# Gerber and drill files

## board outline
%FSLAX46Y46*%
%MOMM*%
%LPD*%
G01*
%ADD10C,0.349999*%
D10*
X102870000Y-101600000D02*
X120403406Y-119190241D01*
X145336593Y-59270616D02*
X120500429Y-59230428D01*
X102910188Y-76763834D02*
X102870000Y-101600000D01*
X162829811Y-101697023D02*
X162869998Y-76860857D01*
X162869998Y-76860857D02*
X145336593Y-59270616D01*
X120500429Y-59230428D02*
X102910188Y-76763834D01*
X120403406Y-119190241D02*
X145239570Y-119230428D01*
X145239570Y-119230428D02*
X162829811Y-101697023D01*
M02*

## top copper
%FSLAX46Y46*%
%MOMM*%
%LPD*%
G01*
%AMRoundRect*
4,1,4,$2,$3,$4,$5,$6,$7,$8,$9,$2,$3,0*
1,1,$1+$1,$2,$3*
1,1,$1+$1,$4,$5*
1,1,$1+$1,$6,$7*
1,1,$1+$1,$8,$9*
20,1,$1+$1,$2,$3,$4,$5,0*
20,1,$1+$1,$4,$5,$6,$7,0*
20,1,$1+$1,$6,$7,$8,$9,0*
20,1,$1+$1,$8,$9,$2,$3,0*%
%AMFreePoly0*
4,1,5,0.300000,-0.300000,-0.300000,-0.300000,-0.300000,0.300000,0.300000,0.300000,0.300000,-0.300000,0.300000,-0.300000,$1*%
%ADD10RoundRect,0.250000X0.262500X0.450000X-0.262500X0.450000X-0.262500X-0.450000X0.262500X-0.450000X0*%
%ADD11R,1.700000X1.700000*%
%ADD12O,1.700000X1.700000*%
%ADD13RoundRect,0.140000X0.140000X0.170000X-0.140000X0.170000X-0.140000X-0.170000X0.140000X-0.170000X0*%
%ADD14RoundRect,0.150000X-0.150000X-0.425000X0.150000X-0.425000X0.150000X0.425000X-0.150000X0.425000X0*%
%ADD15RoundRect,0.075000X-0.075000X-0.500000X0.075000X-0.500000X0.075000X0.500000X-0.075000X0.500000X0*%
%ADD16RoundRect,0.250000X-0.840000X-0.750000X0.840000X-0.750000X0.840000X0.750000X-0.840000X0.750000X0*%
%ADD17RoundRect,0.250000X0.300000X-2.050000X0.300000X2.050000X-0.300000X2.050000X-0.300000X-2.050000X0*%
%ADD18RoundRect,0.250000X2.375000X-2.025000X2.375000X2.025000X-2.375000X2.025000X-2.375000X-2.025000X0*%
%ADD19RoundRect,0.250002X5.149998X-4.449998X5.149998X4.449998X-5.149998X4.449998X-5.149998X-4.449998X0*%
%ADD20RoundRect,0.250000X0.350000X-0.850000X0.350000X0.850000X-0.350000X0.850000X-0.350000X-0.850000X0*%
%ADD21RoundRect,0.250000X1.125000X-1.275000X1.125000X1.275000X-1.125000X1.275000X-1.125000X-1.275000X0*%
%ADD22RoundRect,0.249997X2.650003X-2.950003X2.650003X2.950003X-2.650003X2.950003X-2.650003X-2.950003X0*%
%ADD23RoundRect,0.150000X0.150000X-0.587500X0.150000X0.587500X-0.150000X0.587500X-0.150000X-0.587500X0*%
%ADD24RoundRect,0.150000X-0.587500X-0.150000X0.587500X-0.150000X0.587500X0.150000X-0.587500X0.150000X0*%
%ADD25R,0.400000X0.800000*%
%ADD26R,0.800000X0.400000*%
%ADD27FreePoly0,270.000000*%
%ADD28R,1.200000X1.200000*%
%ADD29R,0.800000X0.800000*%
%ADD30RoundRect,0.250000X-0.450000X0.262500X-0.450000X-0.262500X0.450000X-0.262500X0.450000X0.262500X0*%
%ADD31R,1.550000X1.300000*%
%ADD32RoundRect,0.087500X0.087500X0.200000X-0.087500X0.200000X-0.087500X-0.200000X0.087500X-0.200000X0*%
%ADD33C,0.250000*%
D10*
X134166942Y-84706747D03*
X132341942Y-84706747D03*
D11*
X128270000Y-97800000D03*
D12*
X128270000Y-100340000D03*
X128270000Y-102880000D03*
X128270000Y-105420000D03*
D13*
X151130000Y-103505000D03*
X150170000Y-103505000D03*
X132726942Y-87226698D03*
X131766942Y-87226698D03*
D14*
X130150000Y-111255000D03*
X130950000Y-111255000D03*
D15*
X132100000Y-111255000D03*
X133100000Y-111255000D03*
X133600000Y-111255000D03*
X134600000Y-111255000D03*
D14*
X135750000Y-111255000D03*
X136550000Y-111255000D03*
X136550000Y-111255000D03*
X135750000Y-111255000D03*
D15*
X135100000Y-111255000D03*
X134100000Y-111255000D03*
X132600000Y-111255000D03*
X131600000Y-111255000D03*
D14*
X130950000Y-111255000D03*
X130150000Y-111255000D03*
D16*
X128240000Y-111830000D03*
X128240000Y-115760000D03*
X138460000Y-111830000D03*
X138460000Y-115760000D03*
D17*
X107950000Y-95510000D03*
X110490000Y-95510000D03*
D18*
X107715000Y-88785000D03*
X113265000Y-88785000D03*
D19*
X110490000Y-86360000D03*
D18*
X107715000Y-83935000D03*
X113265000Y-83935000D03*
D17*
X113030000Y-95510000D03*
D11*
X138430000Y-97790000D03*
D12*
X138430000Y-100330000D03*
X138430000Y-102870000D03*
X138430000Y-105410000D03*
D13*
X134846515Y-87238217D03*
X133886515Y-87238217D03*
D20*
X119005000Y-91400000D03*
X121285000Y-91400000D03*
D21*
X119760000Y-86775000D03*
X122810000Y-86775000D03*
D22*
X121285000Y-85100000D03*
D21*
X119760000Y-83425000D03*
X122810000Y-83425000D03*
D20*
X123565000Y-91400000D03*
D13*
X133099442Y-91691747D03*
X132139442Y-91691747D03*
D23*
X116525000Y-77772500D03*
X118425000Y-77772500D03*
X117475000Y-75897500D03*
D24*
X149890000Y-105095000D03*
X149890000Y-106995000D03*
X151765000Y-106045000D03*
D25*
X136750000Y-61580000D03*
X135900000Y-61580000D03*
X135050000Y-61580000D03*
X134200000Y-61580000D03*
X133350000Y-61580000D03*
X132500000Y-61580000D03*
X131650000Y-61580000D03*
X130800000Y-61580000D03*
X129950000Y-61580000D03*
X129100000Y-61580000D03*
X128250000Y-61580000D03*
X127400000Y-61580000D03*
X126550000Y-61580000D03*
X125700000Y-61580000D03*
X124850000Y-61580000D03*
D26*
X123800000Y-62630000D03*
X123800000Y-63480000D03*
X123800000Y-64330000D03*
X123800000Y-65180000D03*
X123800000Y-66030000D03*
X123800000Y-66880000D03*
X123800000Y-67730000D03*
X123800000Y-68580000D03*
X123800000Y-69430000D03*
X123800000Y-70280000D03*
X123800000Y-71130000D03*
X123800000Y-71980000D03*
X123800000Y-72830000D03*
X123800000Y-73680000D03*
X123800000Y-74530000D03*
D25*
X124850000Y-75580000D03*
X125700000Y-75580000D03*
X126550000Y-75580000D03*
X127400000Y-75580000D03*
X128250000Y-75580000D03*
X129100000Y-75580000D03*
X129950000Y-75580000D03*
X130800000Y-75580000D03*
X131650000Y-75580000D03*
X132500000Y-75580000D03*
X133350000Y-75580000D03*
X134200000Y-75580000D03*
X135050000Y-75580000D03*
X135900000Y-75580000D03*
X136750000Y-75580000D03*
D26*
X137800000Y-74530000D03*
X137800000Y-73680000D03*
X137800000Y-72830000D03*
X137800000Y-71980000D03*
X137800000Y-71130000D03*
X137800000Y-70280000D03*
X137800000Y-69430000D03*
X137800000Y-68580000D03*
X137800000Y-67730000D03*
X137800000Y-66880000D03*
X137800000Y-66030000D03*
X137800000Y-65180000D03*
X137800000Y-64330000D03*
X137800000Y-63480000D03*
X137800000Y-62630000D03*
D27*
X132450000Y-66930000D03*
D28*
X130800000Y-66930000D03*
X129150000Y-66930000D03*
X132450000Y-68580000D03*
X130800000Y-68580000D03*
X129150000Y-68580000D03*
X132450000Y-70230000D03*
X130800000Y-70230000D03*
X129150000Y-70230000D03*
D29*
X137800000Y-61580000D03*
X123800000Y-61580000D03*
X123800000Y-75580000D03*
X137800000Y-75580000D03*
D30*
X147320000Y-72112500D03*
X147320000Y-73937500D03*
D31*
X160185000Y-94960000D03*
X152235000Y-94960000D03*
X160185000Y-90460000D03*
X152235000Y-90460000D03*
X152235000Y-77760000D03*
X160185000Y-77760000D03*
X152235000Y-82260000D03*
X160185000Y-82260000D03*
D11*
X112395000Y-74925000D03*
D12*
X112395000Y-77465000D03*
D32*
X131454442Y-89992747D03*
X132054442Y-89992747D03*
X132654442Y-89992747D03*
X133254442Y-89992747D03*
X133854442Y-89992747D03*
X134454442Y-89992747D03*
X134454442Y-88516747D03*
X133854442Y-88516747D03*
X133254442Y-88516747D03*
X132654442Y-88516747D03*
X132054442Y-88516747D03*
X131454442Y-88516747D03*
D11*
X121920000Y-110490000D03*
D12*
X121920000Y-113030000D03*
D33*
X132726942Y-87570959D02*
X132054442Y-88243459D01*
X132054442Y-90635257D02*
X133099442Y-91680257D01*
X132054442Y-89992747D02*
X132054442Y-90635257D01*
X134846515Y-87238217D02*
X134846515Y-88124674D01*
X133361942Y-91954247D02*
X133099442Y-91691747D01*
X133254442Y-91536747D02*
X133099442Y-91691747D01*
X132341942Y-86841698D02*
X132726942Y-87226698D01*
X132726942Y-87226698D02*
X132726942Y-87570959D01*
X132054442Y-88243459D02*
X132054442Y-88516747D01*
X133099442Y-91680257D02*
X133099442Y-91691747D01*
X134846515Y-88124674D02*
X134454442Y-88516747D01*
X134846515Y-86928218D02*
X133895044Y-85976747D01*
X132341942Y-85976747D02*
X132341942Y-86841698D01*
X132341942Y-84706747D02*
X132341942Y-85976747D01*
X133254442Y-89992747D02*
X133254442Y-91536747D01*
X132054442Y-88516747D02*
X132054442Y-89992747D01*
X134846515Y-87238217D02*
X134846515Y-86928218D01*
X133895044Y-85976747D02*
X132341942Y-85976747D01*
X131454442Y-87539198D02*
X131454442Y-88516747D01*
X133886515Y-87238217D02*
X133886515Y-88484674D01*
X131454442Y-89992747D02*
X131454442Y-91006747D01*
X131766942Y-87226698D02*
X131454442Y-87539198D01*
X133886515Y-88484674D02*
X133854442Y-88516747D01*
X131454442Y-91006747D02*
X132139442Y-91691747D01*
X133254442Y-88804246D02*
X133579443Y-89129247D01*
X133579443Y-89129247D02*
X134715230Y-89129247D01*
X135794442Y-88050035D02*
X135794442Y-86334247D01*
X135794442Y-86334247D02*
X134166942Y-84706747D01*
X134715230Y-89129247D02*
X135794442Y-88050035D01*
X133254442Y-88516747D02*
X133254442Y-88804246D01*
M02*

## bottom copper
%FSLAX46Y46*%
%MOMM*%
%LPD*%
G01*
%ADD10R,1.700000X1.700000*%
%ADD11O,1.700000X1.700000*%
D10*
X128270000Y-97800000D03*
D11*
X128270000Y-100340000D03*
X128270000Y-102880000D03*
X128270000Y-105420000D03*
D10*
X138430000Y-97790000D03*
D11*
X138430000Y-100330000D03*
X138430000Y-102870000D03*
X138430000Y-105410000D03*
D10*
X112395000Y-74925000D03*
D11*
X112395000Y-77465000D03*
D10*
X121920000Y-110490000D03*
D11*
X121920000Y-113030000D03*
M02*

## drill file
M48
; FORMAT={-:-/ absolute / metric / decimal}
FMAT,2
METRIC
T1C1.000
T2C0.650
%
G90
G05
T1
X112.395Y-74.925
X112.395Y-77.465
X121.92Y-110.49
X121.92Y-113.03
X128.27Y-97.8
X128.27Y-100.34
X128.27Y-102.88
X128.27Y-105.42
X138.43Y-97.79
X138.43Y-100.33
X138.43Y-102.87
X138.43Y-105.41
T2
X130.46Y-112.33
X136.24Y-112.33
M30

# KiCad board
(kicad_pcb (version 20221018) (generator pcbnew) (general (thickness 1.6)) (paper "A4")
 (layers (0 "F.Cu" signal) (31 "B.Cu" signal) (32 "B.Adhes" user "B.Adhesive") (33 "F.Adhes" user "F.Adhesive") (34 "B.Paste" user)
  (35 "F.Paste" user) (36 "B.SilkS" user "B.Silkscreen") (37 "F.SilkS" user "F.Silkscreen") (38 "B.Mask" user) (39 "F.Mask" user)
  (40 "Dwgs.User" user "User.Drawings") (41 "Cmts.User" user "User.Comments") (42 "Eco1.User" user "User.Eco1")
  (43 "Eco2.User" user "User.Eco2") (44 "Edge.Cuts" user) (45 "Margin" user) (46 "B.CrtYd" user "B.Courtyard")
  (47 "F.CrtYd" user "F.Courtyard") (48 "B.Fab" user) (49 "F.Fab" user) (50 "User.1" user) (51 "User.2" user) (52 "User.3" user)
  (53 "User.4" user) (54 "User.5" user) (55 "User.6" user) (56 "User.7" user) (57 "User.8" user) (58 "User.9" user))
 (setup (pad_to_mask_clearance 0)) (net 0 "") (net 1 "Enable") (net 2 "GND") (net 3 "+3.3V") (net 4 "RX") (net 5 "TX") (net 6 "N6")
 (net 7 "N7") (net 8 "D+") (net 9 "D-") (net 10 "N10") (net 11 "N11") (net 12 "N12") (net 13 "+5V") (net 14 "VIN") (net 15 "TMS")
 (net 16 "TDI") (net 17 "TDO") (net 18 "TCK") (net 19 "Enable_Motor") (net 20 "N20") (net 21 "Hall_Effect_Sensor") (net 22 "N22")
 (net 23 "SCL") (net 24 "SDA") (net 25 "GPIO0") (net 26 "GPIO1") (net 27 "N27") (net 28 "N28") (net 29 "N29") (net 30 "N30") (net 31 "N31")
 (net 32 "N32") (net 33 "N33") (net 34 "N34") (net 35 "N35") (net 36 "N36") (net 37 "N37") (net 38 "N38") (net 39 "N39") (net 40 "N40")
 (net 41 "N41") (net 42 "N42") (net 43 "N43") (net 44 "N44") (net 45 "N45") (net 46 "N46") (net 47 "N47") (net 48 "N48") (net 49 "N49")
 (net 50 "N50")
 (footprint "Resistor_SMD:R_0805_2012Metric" (layer "F.Cu") (at 133.254442 84.706747 180)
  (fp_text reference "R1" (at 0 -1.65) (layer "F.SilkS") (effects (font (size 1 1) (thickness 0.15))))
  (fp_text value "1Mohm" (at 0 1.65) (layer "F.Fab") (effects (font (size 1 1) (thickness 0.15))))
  (pad "1" smd roundrect (at -0.9125 0 180) (size 1.025 1.4) (layers "F.Cu" "F.Paste" "F.Mask") (roundrect_rratio 0.243902) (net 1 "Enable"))
  (pad "2" smd roundrect (at 0.9125 0 180) (size 1.025 1.4) (layers "F.Cu" "F.Paste" "F.Mask") (roundrect_rratio 0.243902) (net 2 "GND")))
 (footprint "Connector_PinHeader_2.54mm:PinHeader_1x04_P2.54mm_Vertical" (layer "F.Cu") (at 128.27 97.8)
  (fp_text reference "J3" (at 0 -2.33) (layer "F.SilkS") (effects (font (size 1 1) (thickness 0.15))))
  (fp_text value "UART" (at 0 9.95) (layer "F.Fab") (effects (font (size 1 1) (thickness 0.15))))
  (pad "1" thru_hole rect (at 0 0) (size 1.7 1.7) (drill 1) (layers "*.Cu" "*.Mask") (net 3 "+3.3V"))
  (pad "2" thru_hole oval (at 0 2.54) (size 1.7 1.7) (drill 1) (layers "*.Cu" "*.Mask") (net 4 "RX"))
  (pad "3" thru_hole oval (at 0 5.08) (size 1.7 1.7) (drill 1) (layers "*.Cu" "*.Mask") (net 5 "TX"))
  (pad "4" thru_hole oval (at 0 7.62) (size 1.7 1.7) (drill 1) (layers "*.Cu" "*.Mask") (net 2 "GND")))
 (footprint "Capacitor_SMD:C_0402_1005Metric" (layer "F.Cu") (at 150.65 103.505 180)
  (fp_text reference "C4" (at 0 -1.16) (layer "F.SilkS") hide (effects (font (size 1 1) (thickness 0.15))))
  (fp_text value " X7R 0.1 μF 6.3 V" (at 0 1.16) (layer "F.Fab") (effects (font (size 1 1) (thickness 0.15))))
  (pad "1" smd roundrect (at -0.48 0 180) (size 0.56 0.62) (layers "F.Cu" "F.Paste" "F.Mask") (roundrect_rratio 0.25) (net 2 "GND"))
  (pad "2" smd roundrect (at 0.48 0 180) (size 0.56 0.62) (layers "F.Cu" "F.Paste" "F.Mask") (roundrect_rratio 0.25) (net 3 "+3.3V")))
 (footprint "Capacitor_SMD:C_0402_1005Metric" (layer "F.Cu") (at 132.246942 87.226698 180)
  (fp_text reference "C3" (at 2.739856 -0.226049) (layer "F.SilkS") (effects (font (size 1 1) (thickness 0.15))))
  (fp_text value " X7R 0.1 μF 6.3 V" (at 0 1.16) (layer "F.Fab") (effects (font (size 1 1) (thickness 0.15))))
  (pad "1" smd roundrect (at -0.48 0 180) (size 0.56 0.62) (layers "F.Cu" "F.Paste" "F.Mask") (roundrect_rratio 0.25) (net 2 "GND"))
  (pad "2" smd roundrect (at 0.48 0 180) (size 0.56 0.62) (layers "F.Cu" "F.Paste" "F.Mask") (roundrect_rratio 0.25) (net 3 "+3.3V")))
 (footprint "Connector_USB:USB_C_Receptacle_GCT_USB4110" (layer "F.Cu") (at 133.35 114.935)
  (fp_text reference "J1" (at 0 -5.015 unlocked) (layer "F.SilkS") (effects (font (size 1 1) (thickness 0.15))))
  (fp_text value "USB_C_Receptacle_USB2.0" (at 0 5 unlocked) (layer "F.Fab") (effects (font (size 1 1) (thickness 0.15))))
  (pad "" np_thru_hole circle (at -2.89 -2.605) (size 0.65 0.65) (drill 0.65) (layers "F&B.Cu" "*.Mask"))
  (pad "" np_thru_hole circle (at 2.89 -2.605) (size 0.65 0.65) (drill 0.65) (layers "F&B.Cu" "*.Mask"))
  (pad "A1" smd roundrect (at -3.2 -3.68) (size 0.6 1.15) (layers "F.Cu" "F.Paste" "F.Mask") (roundrect_rratio 0.25) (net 2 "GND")
   (thermal_bridge_angle 45))
  (pad "A4" smd roundrect (at -2.4 -3.68) (size 0.6 1.15) (layers "F.Cu" "F.Paste" "F.Mask") (roundrect_rratio 0.25) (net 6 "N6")
   (thermal_bridge_angle 45))
  (pad "A5" smd roundrect (at -1.25 -3.68) (size 0.3 1.15) (layers "F.Cu" "F.Paste" "F.Mask") (roundrect_rratio 0.25) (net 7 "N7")
   (thermal_bridge_angle 45))
  (pad "A6" smd roundrect (at -0.25 -3.68) (size 0.3 1.15) (layers "F.Cu" "F.Paste" "F.Mask") (roundrect_rratio 0.25) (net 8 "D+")
   (thermal_bridge_angle 45))
  (pad "A7" smd roundrect (at 0.25 -3.68) (size 0.3 1.15) (layers "F.Cu" "F.Paste" "F.Mask") (roundrect_rratio 0.25) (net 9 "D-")
   (thermal_bridge_angle 45))
  (pad "A8" smd roundrect (at 1.25 -3.68) (size 0.3 1.15) (layers "F.Cu" "F.Paste" "F.Mask") (roundrect_rratio 0.25) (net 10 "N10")
   (thermal_bridge_angle 45))
  (pad "A9" smd roundrect (at 2.4 -3.68) (size 0.6 1.15) (layers "F.Cu" "F.Paste" "F.Mask") (roundrect_rratio 0.25) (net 6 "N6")
   (thermal_bridge_angle 45))
  (pad "A12" smd roundrect (at 3.2 -3.68) (size 0.6 1.15) (layers "F.Cu" "F.Paste" "F.Mask") (roundrect_rratio 0.25) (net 2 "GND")
   (thermal_bridge_angle 45))
  (pad "B1" smd roundrect (at 3.2 -3.68) (size 0.6 1.15) (layers "F.Cu" "F.Paste" "F.Mask") (roundrect_rratio 0.25) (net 2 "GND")
   (thermal_bridge_angle 45))
  (pad "B4" smd roundrect (at 2.4 -3.68) (size 0.6 1.15) (layers "F.Cu" "F.Paste" "F.Mask") (roundrect_rratio 0.25) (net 6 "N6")
   (thermal_bridge_angle 45))
  (pad "B5" smd roundrect (at 1.75 -3.68) (size 0.3 1.15) (layers "F.Cu" "F.Paste" "F.Mask") (roundrect_rratio 0.25) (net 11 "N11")
   (thermal_bridge_angle 45))
  (pad "B6" smd roundrect (at 0.75 -3.68) (size 0.3 1.15) (layers "F.Cu" "F.Paste" "F.Mask") (roundrect_rratio 0.25) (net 8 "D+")
   (thermal_bridge_angle 45))
  (pad "B7" smd roundrect (at -0.75 -3.68) (size 0.3 1.15) (layers "F.Cu" "F.Paste" "F.Mask") (roundrect_rratio 0.25) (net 9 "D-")
   (thermal_bridge_angle 45))
  (pad "B8" smd roundrect (at -1.75 -3.68) (size 0.3 1.15) (layers "F.Cu" "F.Paste" "F.Mask") (roundrect_rratio 0.25) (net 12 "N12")
   (thermal_bridge_angle 45))
  (pad "B9" smd roundrect (at -2.4 -3.68) (size 0.6 1.15) (layers "F.Cu" "F.Paste" "F.Mask") (roundrect_rratio 0.25) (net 6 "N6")
   (thermal_bridge_angle 45))
  (pad "B12" smd roundrect (at -3.2 -3.68) (size 0.6 1.15) (layers "F.Cu" "F.Paste" "F.Mask") (roundrect_rratio 0.25) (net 2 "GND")
   (thermal_bridge_angle 45))
  (pad "S1" smd roundrect (at -5.11 -3.105) (size 2.18 2) (layers "F.Cu" "F.Paste" "F.Mask") (roundrect_rratio 0.125) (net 2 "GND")
   (thermal_bridge_angle 45))
  (pad "S1" smd roundrect (at -5.11 0.825) (size 2.18 2) (layers "F.Cu" "F.Paste" "F.Mask") (roundrect_rratio 0.125) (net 2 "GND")
   (thermal_bridge_angle 45))
  (pad "S1" smd roundrect (at 5.11 -3.105) (size 2.18 2) (layers "F.Cu" "F.Paste" "F.Mask") (roundrect_rratio 0.125) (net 2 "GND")
   (thermal_bridge_angle 45))
  (pad "S1" smd roundrect (at 5.11 0.825) (size 2.18 2) (layers "F.Cu" "F.Paste" "F.Mask") (roundrect_rratio 0.125) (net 2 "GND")
   (thermal_bridge_angle 45)))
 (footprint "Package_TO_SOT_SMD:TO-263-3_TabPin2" (layer "F.Cu") (at 110.49 87.86 90)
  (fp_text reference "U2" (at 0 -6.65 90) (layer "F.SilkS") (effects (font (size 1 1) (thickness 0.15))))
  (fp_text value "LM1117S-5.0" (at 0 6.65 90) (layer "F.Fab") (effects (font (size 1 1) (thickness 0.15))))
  (pad "1" smd roundrect (at -7.65 -2.54 90) (size 4.6 1.1) (layers "F.Cu" "F.Paste" "F.Mask") (roundrect_rratio 0.227273) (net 2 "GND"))
  (pad "2" smd roundrect (at -7.65 0 90) (size 4.6 1.1) (layers "F.Cu" "F.Paste" "F.Mask") (roundrect_rratio 0.227273) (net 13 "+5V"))
  (pad "2" smd roundrect (at -0.925 -2.775 90) (size 4.55 5.25) (layers "F.Cu" "F.Paste") (roundrect_rratio 0.054945) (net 13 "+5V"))
  (pad "2" smd roundrect (at -0.925 2.775 90) (size 4.55 5.25) (layers "F.Cu" "F.Paste") (roundrect_rratio 0.054945) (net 13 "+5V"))
  (pad "2" smd roundrect (at 1.5 0 90) (size 9.4 10.8) (layers "F.Cu" "F.Mask") (roundrect_rratio 0.026596) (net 13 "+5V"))
  (pad "2" smd roundrect (at 3.925 -2.775 90) (size 4.55 5.25) (layers "F.Cu" "F.Paste") (roundrect_rratio 0.054945) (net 13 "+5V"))
  (pad "2" smd roundrect (at 3.925 2.775 90) (size 4.55 5.25) (layers "F.Cu" "F.Paste") (roundrect_rratio 0.054945) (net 13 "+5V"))
  (pad "3" smd roundrect (at -7.65 2.54 90) (size 4.6 1.1) (layers "F.Cu" "F.Paste" "F.Mask") (roundrect_rratio 0.227273) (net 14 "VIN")))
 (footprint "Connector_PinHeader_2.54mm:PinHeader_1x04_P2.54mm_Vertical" (layer "F.Cu") (at 138.43 97.79)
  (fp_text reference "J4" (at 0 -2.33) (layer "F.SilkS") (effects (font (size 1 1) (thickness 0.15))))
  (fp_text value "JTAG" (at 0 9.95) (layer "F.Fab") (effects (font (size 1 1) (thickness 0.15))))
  (pad "1" thru_hole rect (at 0 0) (size 1.7 1.7) (drill 1) (layers "*.Cu" "*.Mask") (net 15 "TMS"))
  (pad "2" thru_hole oval (at 0 2.54) (size 1.7 1.7) (drill 1) (layers "*.Cu" "*.Mask") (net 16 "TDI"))
  (pad "3" thru_hole oval (at 0 5.08) (size 1.7 1.7) (drill 1) (layers "*.Cu" "*.Mask") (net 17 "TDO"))
  (pad "4" thru_hole oval (at 0 7.62) (size 1.7 1.7) (drill 1) (layers "*.Cu" "*.Mask") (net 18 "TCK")))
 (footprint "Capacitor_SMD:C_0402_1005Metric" (layer "F.Cu") (at 134.366515 87.238217 180)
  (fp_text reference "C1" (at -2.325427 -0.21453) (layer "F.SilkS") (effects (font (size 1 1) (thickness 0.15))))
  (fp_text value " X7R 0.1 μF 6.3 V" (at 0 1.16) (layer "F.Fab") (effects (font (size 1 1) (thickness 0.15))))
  (pad "1" smd roundrect (at -0.48 0 180) (size 0.56 0.62) (layers "F.Cu" "F.Paste" "F.Mask") (roundrect_rratio 0.25) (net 2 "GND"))
  (pad "2" smd roundrect (at 0.48 0 180) (size 0.56 0.62) (layers "F.Cu" "F.Paste" "F.Mask") (roundrect_rratio 0.25) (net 3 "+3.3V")))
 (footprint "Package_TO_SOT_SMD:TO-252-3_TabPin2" (layer "F.Cu") (at 121.285 86.36 90)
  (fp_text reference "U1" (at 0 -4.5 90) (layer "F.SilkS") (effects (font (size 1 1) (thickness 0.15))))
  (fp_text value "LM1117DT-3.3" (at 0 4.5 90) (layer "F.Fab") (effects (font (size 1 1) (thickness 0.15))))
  (pad "1" smd roundrect (at -5.04 -2.28 90) (size 2.2 1.2) (layers "F.Cu" "F.Paste" "F.Mask") (roundrect_rratio 0.208333) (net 2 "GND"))
  (pad "2" smd roundrect (at -5.04 0 90) (size 2.2 1.2) (layers "F.Cu" "F.Paste" "F.Mask") (roundrect_rratio 0.208333) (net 3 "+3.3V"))
  (pad "2" smd roundrect (at -0.415 -1.525 90) (size 3.05 2.75) (layers "F.Cu" "F.Paste") (roundrect_rratio 0.090909) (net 3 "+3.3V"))
  (pad "2" smd roundrect (at -0.415 1.525 90) (size 3.05 2.75) (layers "F.Cu" "F.Paste") (roundrect_rratio 0.090909) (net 3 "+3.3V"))
  (pad "2" smd roundrect (at 1.26 0 90) (size 6.4 5.8) (layers "F.Cu" "F.Mask") (roundrect_rratio 0.043103) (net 3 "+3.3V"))
  (pad "2" smd roundrect (at 2.935 -1.525 90) (size 3.05 2.75) (layers "F.Cu" "F.Paste") (roundrect_rratio 0.090909) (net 3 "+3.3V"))
  (pad "2" smd roundrect (at 2.935 1.525 90) (size 3.05 2.75) (layers "F.Cu" "F.Paste") (roundrect_rratio 0.090909) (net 3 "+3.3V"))
  (pad "3" smd roundrect (at -5.04 2.28 90) (size 2.2 1.2) (layers "F.Cu" "F.Paste" "F.Mask") (roundrect_rratio 0.208333) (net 14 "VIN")))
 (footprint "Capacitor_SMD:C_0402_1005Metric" (layer "F.Cu") (at 132.619442 91.691747 180)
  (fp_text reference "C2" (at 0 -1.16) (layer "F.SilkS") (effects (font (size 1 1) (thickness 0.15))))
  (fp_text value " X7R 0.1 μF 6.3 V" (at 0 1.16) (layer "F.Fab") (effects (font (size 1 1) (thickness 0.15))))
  (pad "1" smd roundrect (at -0.48 0 180) (size 0.56 0.62) (layers "F.Cu" "F.Paste" "F.Mask") (roundrect_rratio 0.25) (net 2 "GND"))
  (pad "2" smd roundrect (at 0.48 0 180) (size 0.56 0.62) (layers "F.Cu" "F.Paste" "F.Mask") (roundrect_rratio 0.25) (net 3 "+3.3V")))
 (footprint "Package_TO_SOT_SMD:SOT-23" (layer "F.Cu") (at 117.475 76.835 90)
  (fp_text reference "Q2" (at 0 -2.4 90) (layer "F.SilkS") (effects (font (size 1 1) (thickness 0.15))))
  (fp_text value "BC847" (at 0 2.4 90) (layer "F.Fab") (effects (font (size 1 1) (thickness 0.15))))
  (pad "1" smd roundrect (at -0.9375 -0.95 90) (size 1.475 0.6) (layers "F.Cu" "F.Paste" "F.Mask") (roundrect_rratio 0.25)
   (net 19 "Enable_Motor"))
  (pad "2" smd roundrect (at -0.9375 0.95 90) (size 1.475 0.6) (layers "F.Cu" "F.Paste" "F.Mask") (roundrect_rratio 0.25) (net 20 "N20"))
  (pad "3" smd roundrect (at 0.9375 0 90) (size 1.475 0.6) (layers "F.Cu" "F.Paste" "F.Mask") (roundrect_rratio 0.25) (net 2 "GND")))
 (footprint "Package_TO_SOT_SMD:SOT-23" (layer "F.Cu") (at 150.8275 106.045)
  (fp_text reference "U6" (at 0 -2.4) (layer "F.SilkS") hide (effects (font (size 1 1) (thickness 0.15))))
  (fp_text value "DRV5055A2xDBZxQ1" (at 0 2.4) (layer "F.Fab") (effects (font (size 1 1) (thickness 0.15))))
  (pad "1" smd roundrect (at -0.9375 -0.95) (size 1.475 0.6) (layers "F.Cu" "F.Paste" "F.Mask") (roundrect_rratio 0.25) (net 3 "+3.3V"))
  (pad "2" smd roundrect (at -0.9375 0.95) (size 1.475 0.6) (layers "F.Cu" "F.Paste" "F.Mask") (roundrect_rratio 0.25)
   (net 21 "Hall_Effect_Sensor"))
  (pad "3" smd roundrect (at 0.9375 0) (size 1.475 0.6) (layers "F.Cu" "F.Paste" "F.Mask") (roundrect_rratio 0.25) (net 2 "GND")))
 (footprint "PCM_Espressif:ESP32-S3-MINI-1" (layer "F.Cu") (at 130.8 68.58 -90)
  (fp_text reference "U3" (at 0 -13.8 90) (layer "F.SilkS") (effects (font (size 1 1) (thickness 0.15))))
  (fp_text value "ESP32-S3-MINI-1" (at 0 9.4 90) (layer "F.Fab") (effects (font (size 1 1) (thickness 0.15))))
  (pad "1" smd rect (at -7 -5.95) (size 0.4 0.8) (layers "F.Cu" "F.Paste" "F.Mask") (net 2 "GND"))
  (pad "2" smd rect (at -7 -5.1) (size 0.4 0.8) (layers "F.Cu" "F.Paste" "F.Mask") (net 2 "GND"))
  (pad "3" smd rect (at -7 -4.25) (size 0.4 0.8) (layers "F.Cu" "F.Paste" "F.Mask") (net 3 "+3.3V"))
  (pad "4" smd rect (at -7 -3.4) (size 0.4 0.8) (layers "F.Cu" "F.Paste" "F.Mask") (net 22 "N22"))
  (pad "5" smd rect (at -7 -2.55) (size 0.4 0.8) (layers "F.Cu" "F.Paste" "F.Mask") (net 1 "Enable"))
  (pad "6" smd rect (at -7 -1.7) (size 0.4 0.8) (layers "F.Cu" "F.Paste" "F.Mask") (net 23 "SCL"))
  (pad "7" smd rect (at -7 -0.85) (size 0.4 0.8) (layers "F.Cu" "F.Paste" "F.Mask") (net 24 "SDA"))
  (pad "8" smd rect (at -7 0) (size 0.4 0.8) (layers "F.Cu" "F.Paste" "F.Mask") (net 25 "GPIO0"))
  (pad "9" smd rect (at -7 0.85) (size 0.4 0.8) (layers "F.Cu" "F.Paste" "F.Mask") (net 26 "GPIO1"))
  (pad "10" smd rect (at -7 1.7) (size 0.4 0.8) (layers "F.Cu" "F.Paste" "F.Mask") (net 19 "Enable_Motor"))
  (pad "11" smd rect (at -7 2.55) (size 0.4 0.8) (layers "F.Cu" "F.Paste" "F.Mask") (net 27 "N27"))
  (pad "12" smd rect (at -7 3.4) (size 0.4 0.8) (layers "F.Cu" "F.Paste" "F.Mask") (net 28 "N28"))
  (pad "13" smd rect (at -7 4.25) (size 0.4 0.8) (layers "F.Cu" "F.Paste" "F.Mask") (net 21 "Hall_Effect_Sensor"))
  (pad "14" smd rect (at -7 5.1) (size 0.4 0.8) (layers "F.Cu" "F.Paste" "F.Mask") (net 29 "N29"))
  (pad "15" smd rect (at -7 5.95) (size 0.4 0.8) (layers "F.Cu" "F.Paste" "F.Mask") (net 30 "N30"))
  (pad "16" smd rect (at -5.95 7 270) (size 0.4 0.8) (layers "F.Cu" "F.Paste" "F.Mask") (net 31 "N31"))
  (pad "17" smd rect (at -5.1 7 270) (size 0.4 0.8) (layers "F.Cu" "F.Paste" "F.Mask") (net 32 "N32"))
  (pad "18" smd rect (at -4.25 7 270) (size 0.4 0.8) (layers "F.Cu" "F.Paste" "F.Mask") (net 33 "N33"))
  (pad "19" smd rect (at -3.4 7 270) (size 0.4 0.8) (layers "F.Cu" "F.Paste" "F.Mask") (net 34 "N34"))
  (pad "20" smd rect (at -2.55 7 270) (size 0.4 0.8) (layers "F.Cu" "F.Paste" "F.Mask") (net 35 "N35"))
  (pad "21" smd rect (at -1.7 7 270) (size 0.4 0.8) (layers "F.Cu" "F.Paste" "F.Mask") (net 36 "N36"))
  (pad "22" smd rect (at -0.85 7 270) (size 0.4 0.8) (layers "F.Cu" "F.Paste" "F.Mask") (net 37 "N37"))
  (pad "23" smd rect (at 0 7 270) (size 0.4 0.8) (layers "F.Cu" "F.Paste" "F.Mask") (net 9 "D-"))
  (pad "24" smd rect (at 0.85 7 270) (size 0.4 0.8) (layers "F.Cu" "F.Paste" "F.Mask") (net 8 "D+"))
  (pad "25" smd rect (at 1.7 7 270) (size 0.4 0.8) (layers "F.Cu" "F.Paste" "F.Mask") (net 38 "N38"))
  (pad "26" smd rect (at 2.55 7 270) (size 0.4 0.8) (layers "F.Cu" "F.Paste" "F.Mask") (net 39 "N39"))
  (pad "27" smd rect (at 3.4 7 270) (size 0.4 0.8) (layers "F.Cu" "F.Paste" "F.Mask") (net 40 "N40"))
  (pad "28" smd rect (at 4.25 7 270) (size 0.4 0.8) (layers "F.Cu" "F.Paste" "F.Mask") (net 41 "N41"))
  (pad "29" smd rect (at 5.1 7 270) (size 0.4 0.8) (layers "F.Cu" "F.Paste" "F.Mask") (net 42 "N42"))
  (pad "30" smd rect (at 5.95 7 270) (size 0.4 0.8) (layers "F.Cu" "F.Paste" "F.Mask") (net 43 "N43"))
  (pad "31" smd rect (at 7 5.95) (size 0.4 0.8) (layers "F.Cu" "F.Paste" "F.Mask") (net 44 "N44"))
  (pad "32" smd rect (at 7 5.1) (size 0.4 0.8) (layers "F.Cu" "F.Paste" "F.Mask") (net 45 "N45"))
  (pad "33" smd rect (at 7 4.25) (size 0.4 0.8) (layers "F.Cu" "F.Paste" "F.Mask") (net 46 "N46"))
  (pad "34" smd rect (at 7 3.4) (size 0.4 0.8) (layers "F.Cu" "F.Paste" "F.Mask") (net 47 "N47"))
  (pad "35" smd rect (at 7 2.55) (size 0.4 0.8) (layers "F.Cu" "F.Paste" "F.Mask") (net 18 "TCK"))
  (pad "36" smd rect (at 7 1.7) (size 0.4 0.8) (layers "F.Cu" "F.Paste" "F.Mask") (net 17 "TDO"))
  (pad "37" smd rect (at 7 0.85) (size 0.4 0.8) (layers "F.Cu" "F.Paste" "F.Mask") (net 16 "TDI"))
  (pad "38" smd rect (at 7 0) (size 0.4 0.8) (layers "F.Cu" "F.Paste" "F.Mask") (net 15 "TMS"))
  (pad "39" smd rect (at 7 -0.85) (size 0.4 0.8) (layers "F.Cu" "F.Paste" "F.Mask") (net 5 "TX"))
  (pad "40" smd rect (at 7 -1.7) (size 0.4 0.8) (layers "F.Cu" "F.Paste" "F.Mask") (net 4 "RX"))
  (pad "41" smd rect (at 7 -2.55) (size 0.4 0.8) (layers "F.Cu" "F.Paste" "F.Mask") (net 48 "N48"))
  (pad "42" smd rect (at 7 -3.4) (size 0.4 0.8) (layers "F.Cu" "F.Paste" "F.Mask") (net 2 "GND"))
  (pad "43" smd rect (at 7 -4.25) (size 0.4 0.8) (layers "F.Cu" "F.Paste" "F.Mask") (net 2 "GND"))
  (pad "44" smd rect (at 7 -5.1) (size 0.4 0.8) (layers "F.Cu" "F.Paste" "F.Mask") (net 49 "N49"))
  (pad "45" smd rect (at 7 -5.95) (size 0.4 0.8) (layers "F.Cu" "F.Paste" "F.Mask") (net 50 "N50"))
  (pad "46" smd rect (at 5.95 -7 270) (size 0.4 0.8) (layers "F.Cu" "F.Paste" "F.Mask") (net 2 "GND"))
  (pad "47" smd rect (at 5.1 -7 270) (size 0.4 0.8) (layers "F.Cu" "F.Paste" "F.Mask") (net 2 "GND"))
  (pad "48" smd rect (at 4.25 -7 270) (size 0.4 0.8) (layers "F.Cu" "F.Paste" "F.Mask") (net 2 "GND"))
  (pad "49" smd rect (at 3.4 -7 270) (size 0.4 0.8) (layers "F.Cu" "F.Paste" "F.Mask") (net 2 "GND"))
  (pad "50" smd rect (at 2.55 -7 270) (size 0.4 0.8) (layers "F.Cu" "F.Paste" "F.Mask") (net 2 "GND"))
  (pad "51" smd rect (at 1.7 -7 270) (size 0.4 0.8) (layers "F.Cu" "F.Paste" "F.Mask") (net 2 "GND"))
  (pad "52" smd rect (at 0.85 -7 270) (size 0.4 0.8) (layers "F.Cu" "F.Paste" "F.Mask") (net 2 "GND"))
  (pad "53" smd rect (at 0 -7 270) (size 0.4 0.8) (layers "F.Cu" "F.Paste" "F.Mask") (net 2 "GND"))
  (pad "54" smd rect (at -0.85 -7 270) (size 0.4 0.8) (layers "F.Cu" "F.Paste" "F.Mask") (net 2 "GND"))
  (pad "55" smd rect (at -1.7 -7 270) (size 0.4 0.8) (layers "F.Cu" "F.Paste" "F.Mask") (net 2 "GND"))
  (pad "56" smd rect (at -2.55 -7 270) (size 0.4 0.8) (layers "F.Cu" "F.Paste" "F.Mask") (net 2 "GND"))
  (pad "57" smd rect (at -3.4 -7 270) (size 0.4 0.8) (layers "F.Cu" "F.Paste" "F.Mask") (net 2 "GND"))
  (pad "58" smd rect (at -4.25 -7 270) (size 0.4 0.8) (layers "F.Cu" "F.Paste" "F.Mask") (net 2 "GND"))
  (pad "59" smd rect (at -5.1 -7 270) (size 0.4 0.8) (layers "F.Cu" "F.Paste" "F.Mask") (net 2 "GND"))
  (pad "60" smd rect (at -5.95 -7 270) (size 0.4 0.8) (layers "F.Cu" "F.Paste" "F.Mask") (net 2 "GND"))
  (pad "61" smd custom (at -1.65 -1.65 270) (size 0.6 0.6) (layers "F.Cu" "F.Paste" "F.Mask") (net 2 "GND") (zone_connect 2)
   (thermal_bridge_angle 45) (options (clearance outline) (anchor rect)) (primitives))
  (pad "61" smd rect (at -1.65 0 270) (size 1.2 1.2) (layers "F.Cu" "F.Paste" "F.Mask") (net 2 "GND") (zone_connect 2))
  (pad "61" smd rect (at -1.65 1.65 270) (size 1.2 1.2) (layers "F.Cu" "F.Paste" "F.Mask") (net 2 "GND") (zone_connect 2))
  (pad "61" smd rect (at 0 -1.65 270) (size 1.2 1.2) (layers "F.Cu" "F.Paste" "F.Mask") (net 2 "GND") (zone_connect 2))
  (pad "61" smd rect (at 0 0 270) (size 1.2 1.2) (layers "F.Cu" "F.Paste" "F.Mask") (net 2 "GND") (zone_connect 2))
  (pad "61" smd rect (at 0 1.65 270) (size 1.2 1.2) (layers "F.Cu" "F.Paste" "F.Mask") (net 2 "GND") (zone_connect 2))
  (pad "61" smd rect (at 1.65 -1.65 270) (size 1.2 1.2) (layers "F.Cu" "F.Paste" "F.Mask") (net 2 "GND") (zone_connect 2))
  (pad "61" smd rect (at 1.65 0 270) (size 1.2 1.2) (layers "F.Cu" "F.Paste" "F.Mask") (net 2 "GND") (zone_connect 2))
  (pad "61" smd rect (at 1.65 1.65 270) (size 1.2 1.2) (layers "F.Cu" "F.Paste" "F.Mask") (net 2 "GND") (zone_connect 2))
  (pad "62" smd rect (at -7 -7 90) (size 0.8 0.8) (layers "F.Cu" "F.Paste" "F.Mask") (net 2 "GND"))
  (pad "63" smd rect (at -7 7 90) (size 0.8 0.8) (layers "F.Cu" "F.Paste" "F.Mask") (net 2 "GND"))
  (pad "64" smd rect (at 7 7 90) (size 0.8 0.8) (layers "F.Cu" "F.Paste" "F.Mask") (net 2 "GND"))
  (pad "65" smd rect (at 7 -7 90) (size 0.8 0.8) (layers "F.Cu" "F.Paste" "F.Mask") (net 2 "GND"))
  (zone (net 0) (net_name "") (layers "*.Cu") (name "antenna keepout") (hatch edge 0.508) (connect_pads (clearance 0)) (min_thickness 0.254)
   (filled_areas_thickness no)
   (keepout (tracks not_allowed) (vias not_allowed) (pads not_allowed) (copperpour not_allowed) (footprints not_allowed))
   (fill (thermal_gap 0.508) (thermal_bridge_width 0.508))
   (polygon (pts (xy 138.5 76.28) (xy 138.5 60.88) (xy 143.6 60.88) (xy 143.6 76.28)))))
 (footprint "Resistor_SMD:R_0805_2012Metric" (layer "F.Cu") (at 147.32 73.025 -90)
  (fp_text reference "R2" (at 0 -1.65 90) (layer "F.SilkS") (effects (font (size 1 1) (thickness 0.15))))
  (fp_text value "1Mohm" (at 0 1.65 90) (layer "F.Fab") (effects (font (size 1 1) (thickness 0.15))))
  (pad "1" smd roundrect (at -0.9125 0 270) (size 1.025 1.4) (layers "F.Cu" "F.Paste" "F.Mask") (roundrect_rratio 0.243902)
   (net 19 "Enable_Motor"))
  (pad "2" smd roundrect (at 0.9125 0 270) (size 1.025 1.4) (layers "F.Cu" "F.Paste" "F.Mask") (roundrect_rratio 0.243902) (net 2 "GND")))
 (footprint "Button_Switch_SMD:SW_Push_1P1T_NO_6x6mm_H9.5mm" (layer "F.Cu") (at 156.21 92.71 180)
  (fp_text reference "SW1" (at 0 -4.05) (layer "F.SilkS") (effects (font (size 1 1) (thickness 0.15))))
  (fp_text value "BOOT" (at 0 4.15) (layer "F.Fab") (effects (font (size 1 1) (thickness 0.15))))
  (pad "1" smd rect (at -3.975 -2.25 180) (size 1.55 1.3) (layers "F.Cu" "F.Paste" "F.Mask") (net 2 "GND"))
  (pad "1" smd rect (at 3.975 -2.25 180) (size 1.55 1.3) (layers "F.Cu" "F.Paste" "F.Mask") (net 2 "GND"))
  (pad "2" smd rect (at -3.975 2.25 180) (size 1.55 1.3) (layers "F.Cu" "F.Paste" "F.Mask") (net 22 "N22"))
  (pad "2" smd rect (at 3.975 2.25 180) (size 1.55 1.3) (layers "F.Cu" "F.Paste" "F.Mask") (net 22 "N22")))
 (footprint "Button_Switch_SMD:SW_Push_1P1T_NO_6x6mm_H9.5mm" (layer "F.Cu") (at 156.21 80.01)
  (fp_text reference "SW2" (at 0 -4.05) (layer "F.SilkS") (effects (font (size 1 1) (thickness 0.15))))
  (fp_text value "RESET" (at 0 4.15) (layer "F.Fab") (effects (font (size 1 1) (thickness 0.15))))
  (pad "1" smd rect (at -3.975 -2.25) (size 1.55 1.3) (layers "F.Cu" "F.Paste" "F.Mask") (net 50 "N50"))
  (pad "1" smd rect (at 3.975 -2.25) (size 1.55 1.3) (layers "F.Cu" "F.Paste" "F.Mask") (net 50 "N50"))
  (pad "2" smd rect (at -3.975 2.25) (size 1.55 1.3) (layers "F.Cu" "F.Paste" "F.Mask") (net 3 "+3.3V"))
  (pad "2" smd rect (at 3.975 2.25) (size 1.55 1.3) (layers "F.Cu" "F.Paste" "F.Mask") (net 3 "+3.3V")))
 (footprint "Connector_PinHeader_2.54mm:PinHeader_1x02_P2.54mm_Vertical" (layer "F.Cu") (at 112.395 74.925)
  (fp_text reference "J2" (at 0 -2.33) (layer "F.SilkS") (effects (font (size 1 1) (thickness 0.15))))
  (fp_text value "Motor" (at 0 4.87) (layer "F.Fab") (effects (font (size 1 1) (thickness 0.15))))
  (pad "1" thru_hole rect (at 0 0) (size 1.7 1.7) (drill 1) (layers "*.Cu" "*.Mask") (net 20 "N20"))
  (pad "2" thru_hole oval (at 0 2.54) (size 1.7 1.7) (drill 1) (layers "*.Cu" "*.Mask") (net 13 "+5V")))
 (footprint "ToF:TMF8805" (layer "F.Cu") (at 132.951299 82.893217)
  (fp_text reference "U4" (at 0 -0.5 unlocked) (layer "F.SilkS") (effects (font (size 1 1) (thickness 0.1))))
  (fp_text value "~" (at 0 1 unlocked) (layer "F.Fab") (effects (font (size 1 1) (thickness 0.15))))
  (pad "1" smd roundrect (at -1.496857 7.09953 180) (size 0.35 0.575) (layers "F.Cu" "F.Paste" "F.Mask") (roundrect_rratio 0.25)
   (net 3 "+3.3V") (thermal_bridge_angle 45))
  (pad "2" smd roundrect (at -0.896857 7.09953 180) (size 0.35 0.575) (layers "F.Cu" "F.Paste" "F.Mask") (roundrect_rratio 0.25)
   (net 2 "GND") (thermal_bridge_angle 45))
  (pad "3" smd roundrect (at -0.296857 7.09953 180) (size 0.35 0.575) (layers "F.Cu" "F.Paste" "F.Mask") (roundrect_rratio 0.25)
   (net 26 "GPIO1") (thermal_bridge_angle 45))
  (pad "4" smd roundrect (at 0.303143 7.09953 180) (size 0.35 0.575) (layers "F.Cu" "F.Paste" "F.Mask") (roundrect_rratio 0.25)
   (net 2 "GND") (thermal_bridge_angle 45))
  (pad "5" smd roundrect (at 0.903143 7.09953 180) (size 0.35 0.575) (layers "F.Cu" "F.Paste" "F.Mask") (roundrect_rratio 0.25)
   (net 23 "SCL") (thermal_bridge_angle 45))
  (pad "6" smd roundrect (at 1.503143 7.09953 180) (size 0.35 0.575) (layers "F.Cu" "F.Paste" "F.Mask") (roundrect_rratio 0.25)
   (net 24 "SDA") (thermal_bridge_angle 45))
  (pad "7" smd roundrect (at 1.503143 5.62353 180) (size 0.35 0.575) (layers "F.Cu" "F.Paste" "F.Mask") (roundrect_rratio 0.25)
   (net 2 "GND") (thermal_bridge_angle 45))
  (pad "8" smd roundrect (at 0.903143 5.62353 180) (size 0.35 0.575) (layers "F.Cu" "F.Paste" "F.Mask") (roundrect_rratio 0.25)
   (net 3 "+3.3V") (thermal_bridge_angle 45))
  (pad "9" smd roundrect (at 0.303143 5.62353 180) (size 0.35 0.575) (layers "F.Cu" "F.Paste" "F.Mask") (roundrect_rratio 0.25)
   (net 1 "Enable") (thermal_bridge_angle 45))
  (pad "10" smd roundrect (at -0.296857 5.62353 180) (size 0.35 0.575) (layers "F.Cu" "F.Paste" "F.Mask") (roundrect_rratio 0.25)
   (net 25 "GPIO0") (thermal_bridge_angle 45))
  (pad "11" smd roundrect (at -0.896857 5.62353 180) (size 0.35 0.575) (layers "F.Cu" "F.Paste" "F.Mask") (roundrect_rratio 0.25)
   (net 2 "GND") (thermal_bridge_angle 45))
  (pad "12" smd roundrect (at -1.496857 5.62353 180) (size 0.35 0.575) (layers "F.Cu" "F.Paste" "F.Mask") (roundrect_rratio 0.25)
   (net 3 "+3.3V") (thermal_bridge_angle 45)))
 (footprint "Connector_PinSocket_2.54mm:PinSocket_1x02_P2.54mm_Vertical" (layer "F.Cu") (at 121.92 110.49)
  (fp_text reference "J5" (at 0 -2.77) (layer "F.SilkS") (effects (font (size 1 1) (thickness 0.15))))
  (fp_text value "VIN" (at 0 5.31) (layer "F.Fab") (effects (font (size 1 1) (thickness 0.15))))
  (pad "1" thru_hole rect (at 0 0) (size 1.7 1.7) (drill 1) (layers "*.Cu" "*.Mask") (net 14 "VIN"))
  (pad "2" thru_hole oval (at 0 2.54) (size 1.7 1.7) (drill 1) (layers "*.Cu" "*.Mask") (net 2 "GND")))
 (gr_line (start 102.87 101.6) (end 120.403406 119.190241) (stroke (width 0.349999) (type solid)) (layer "Edge.Cuts"))
 (gr_line (start 145.336593 59.270616) (end 120.500429 59.230428) (stroke (width 0.349999) (type solid)) (layer "Edge.Cuts"))
 (gr_line (start 102.910188 76.763834) (end 102.87 101.6) (stroke (width 0.349999) (type solid)) (layer "Edge.Cuts"))
 (gr_line (start 162.829811 101.697023) (end 162.869998 76.860857) (stroke (width 0.349999) (type solid)) (layer "Edge.Cuts"))
 (gr_line (start 162.869998 76.860857) (end 145.336593 59.270616) (stroke (width 0.349999) (type solid)) (layer "Edge.Cuts"))
 (gr_line (start 120.500429 59.230428) (end 102.910188 76.763834) (stroke (width 0.349999) (type solid)) (layer "Edge.Cuts"))
 (gr_line (start 120.403406 119.190241) (end 145.23957 119.230428) (stroke (width 0.349999) (type solid)) (layer "Edge.Cuts"))
 (gr_line (start 145.23957 119.230428) (end 162.829811 101.697023) (stroke (width 0.349999) (type solid)) (layer "Edge.Cuts"))
 (segment (start 132.726942 87.570959) (end 132.054442 88.243459) (width 0.25) (layer "F.Cu") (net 2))
 (segment (start 132.054442 90.635257) (end 133.099442 91.680257) (width 0.25) (layer "F.Cu") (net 2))
 (segment (start 132.054442 89.992747) (end 132.054442 90.635257) (width 0.25) (layer "F.Cu") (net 2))
 (segment (start 134.846515 87.238217) (end 134.846515 88.124674) (width 0.25) (layer "F.Cu") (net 2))
 (segment (start 133.361942 91.954247) (end 133.099442 91.691747) (width 0.25) (layer "F.Cu") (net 2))
 (segment (start 133.254442 91.536747) (end 133.099442 91.691747) (width 0.25) (layer "F.Cu") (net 2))
 (segment (start 132.341942 86.841698) (end 132.726942 87.226698) (width 0.25) (layer "F.Cu") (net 2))
 (segment (start 132.726942 87.226698) (end 132.726942 87.570959) (width 0.25) (layer "F.Cu") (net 2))
 (segment (start 132.054442 88.243459) (end 132.054442 88.516747) (width 0.25) (layer "F.Cu") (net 2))
 (segment (start 133.099442 91.680257) (end 133.099442 91.691747) (width 0.25) (layer "F.Cu") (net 2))
 (segment (start 134.846515 88.124674) (end 134.454442 88.516747) (width 0.25) (layer "F.Cu") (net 2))
 (segment (start 134.846515 86.928218) (end 133.895044 85.976747) (width 0.25) (layer "F.Cu") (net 2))
 (segment (start 132.341942 85.976747) (end 132.341942 86.841698) (width 0.25) (layer "F.Cu") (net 2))
 (segment (start 132.341942 84.706747) (end 132.341942 85.976747) (width 0.25) (layer "F.Cu") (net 2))
 (segment (start 133.254442 89.992747) (end 133.254442 91.536747) (width 0.25) (layer "F.Cu") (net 2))
 (segment (start 132.054442 88.516747) (end 132.054442 89.992747) (width 0.25) (layer "F.Cu") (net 2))
 (segment (start 134.846515 87.238217) (end 134.846515 86.928218) (width 0.25) (layer "F.Cu") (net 2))
 (segment (start 133.895044 85.976747) (end 132.341942 85.976747) (width 0.25) (layer "F.Cu") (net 2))
 (segment (start 131.454442 87.539198) (end 131.454442 88.516747) (width 0.25) (layer "F.Cu") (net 3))
 (segment (start 133.886515 87.238217) (end 133.886515 88.484674) (width 0.25) (layer "F.Cu") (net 3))
 (segment (start 131.454442 89.992747) (end 131.454442 91.006747) (width 0.25) (layer "F.Cu") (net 3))
 (segment (start 131.766942 87.226698) (end 131.454442 87.539198) (width 0.25) (layer "F.Cu") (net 3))
 (segment (start 133.886515 88.484674) (end 133.854442 88.516747) (width 0.25) (layer "F.Cu") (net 3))
 (segment (start 131.454442 91.006747) (end 132.139442 91.691747) (width 0.25) (layer "F.Cu") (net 3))
 (segment (start 133.254442 88.804246) (end 133.579443 89.129247) (width 0.25) (layer "F.Cu") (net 1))
 (segment (start 133.579443 89.129247) (end 134.71523 89.129247) (width 0.25) (layer "F.Cu") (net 1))
 (segment (start 135.794442 88.050035) (end 135.794442 86.334247) (width 0.25) (layer "F.Cu") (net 1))
 (segment (start 135.794442 86.334247) (end 134.166942 84.706747) (width 0.25) (layer "F.Cu") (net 1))
 (segment (start 134.71523 89.129247) (end 135.794442 88.050035) (width 0.25) (layer "F.Cu") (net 1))
 (segment (start 133.254442 88.516747) (end 133.254442 88.804246) (width 0.25) (layer "F.Cu") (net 1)))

